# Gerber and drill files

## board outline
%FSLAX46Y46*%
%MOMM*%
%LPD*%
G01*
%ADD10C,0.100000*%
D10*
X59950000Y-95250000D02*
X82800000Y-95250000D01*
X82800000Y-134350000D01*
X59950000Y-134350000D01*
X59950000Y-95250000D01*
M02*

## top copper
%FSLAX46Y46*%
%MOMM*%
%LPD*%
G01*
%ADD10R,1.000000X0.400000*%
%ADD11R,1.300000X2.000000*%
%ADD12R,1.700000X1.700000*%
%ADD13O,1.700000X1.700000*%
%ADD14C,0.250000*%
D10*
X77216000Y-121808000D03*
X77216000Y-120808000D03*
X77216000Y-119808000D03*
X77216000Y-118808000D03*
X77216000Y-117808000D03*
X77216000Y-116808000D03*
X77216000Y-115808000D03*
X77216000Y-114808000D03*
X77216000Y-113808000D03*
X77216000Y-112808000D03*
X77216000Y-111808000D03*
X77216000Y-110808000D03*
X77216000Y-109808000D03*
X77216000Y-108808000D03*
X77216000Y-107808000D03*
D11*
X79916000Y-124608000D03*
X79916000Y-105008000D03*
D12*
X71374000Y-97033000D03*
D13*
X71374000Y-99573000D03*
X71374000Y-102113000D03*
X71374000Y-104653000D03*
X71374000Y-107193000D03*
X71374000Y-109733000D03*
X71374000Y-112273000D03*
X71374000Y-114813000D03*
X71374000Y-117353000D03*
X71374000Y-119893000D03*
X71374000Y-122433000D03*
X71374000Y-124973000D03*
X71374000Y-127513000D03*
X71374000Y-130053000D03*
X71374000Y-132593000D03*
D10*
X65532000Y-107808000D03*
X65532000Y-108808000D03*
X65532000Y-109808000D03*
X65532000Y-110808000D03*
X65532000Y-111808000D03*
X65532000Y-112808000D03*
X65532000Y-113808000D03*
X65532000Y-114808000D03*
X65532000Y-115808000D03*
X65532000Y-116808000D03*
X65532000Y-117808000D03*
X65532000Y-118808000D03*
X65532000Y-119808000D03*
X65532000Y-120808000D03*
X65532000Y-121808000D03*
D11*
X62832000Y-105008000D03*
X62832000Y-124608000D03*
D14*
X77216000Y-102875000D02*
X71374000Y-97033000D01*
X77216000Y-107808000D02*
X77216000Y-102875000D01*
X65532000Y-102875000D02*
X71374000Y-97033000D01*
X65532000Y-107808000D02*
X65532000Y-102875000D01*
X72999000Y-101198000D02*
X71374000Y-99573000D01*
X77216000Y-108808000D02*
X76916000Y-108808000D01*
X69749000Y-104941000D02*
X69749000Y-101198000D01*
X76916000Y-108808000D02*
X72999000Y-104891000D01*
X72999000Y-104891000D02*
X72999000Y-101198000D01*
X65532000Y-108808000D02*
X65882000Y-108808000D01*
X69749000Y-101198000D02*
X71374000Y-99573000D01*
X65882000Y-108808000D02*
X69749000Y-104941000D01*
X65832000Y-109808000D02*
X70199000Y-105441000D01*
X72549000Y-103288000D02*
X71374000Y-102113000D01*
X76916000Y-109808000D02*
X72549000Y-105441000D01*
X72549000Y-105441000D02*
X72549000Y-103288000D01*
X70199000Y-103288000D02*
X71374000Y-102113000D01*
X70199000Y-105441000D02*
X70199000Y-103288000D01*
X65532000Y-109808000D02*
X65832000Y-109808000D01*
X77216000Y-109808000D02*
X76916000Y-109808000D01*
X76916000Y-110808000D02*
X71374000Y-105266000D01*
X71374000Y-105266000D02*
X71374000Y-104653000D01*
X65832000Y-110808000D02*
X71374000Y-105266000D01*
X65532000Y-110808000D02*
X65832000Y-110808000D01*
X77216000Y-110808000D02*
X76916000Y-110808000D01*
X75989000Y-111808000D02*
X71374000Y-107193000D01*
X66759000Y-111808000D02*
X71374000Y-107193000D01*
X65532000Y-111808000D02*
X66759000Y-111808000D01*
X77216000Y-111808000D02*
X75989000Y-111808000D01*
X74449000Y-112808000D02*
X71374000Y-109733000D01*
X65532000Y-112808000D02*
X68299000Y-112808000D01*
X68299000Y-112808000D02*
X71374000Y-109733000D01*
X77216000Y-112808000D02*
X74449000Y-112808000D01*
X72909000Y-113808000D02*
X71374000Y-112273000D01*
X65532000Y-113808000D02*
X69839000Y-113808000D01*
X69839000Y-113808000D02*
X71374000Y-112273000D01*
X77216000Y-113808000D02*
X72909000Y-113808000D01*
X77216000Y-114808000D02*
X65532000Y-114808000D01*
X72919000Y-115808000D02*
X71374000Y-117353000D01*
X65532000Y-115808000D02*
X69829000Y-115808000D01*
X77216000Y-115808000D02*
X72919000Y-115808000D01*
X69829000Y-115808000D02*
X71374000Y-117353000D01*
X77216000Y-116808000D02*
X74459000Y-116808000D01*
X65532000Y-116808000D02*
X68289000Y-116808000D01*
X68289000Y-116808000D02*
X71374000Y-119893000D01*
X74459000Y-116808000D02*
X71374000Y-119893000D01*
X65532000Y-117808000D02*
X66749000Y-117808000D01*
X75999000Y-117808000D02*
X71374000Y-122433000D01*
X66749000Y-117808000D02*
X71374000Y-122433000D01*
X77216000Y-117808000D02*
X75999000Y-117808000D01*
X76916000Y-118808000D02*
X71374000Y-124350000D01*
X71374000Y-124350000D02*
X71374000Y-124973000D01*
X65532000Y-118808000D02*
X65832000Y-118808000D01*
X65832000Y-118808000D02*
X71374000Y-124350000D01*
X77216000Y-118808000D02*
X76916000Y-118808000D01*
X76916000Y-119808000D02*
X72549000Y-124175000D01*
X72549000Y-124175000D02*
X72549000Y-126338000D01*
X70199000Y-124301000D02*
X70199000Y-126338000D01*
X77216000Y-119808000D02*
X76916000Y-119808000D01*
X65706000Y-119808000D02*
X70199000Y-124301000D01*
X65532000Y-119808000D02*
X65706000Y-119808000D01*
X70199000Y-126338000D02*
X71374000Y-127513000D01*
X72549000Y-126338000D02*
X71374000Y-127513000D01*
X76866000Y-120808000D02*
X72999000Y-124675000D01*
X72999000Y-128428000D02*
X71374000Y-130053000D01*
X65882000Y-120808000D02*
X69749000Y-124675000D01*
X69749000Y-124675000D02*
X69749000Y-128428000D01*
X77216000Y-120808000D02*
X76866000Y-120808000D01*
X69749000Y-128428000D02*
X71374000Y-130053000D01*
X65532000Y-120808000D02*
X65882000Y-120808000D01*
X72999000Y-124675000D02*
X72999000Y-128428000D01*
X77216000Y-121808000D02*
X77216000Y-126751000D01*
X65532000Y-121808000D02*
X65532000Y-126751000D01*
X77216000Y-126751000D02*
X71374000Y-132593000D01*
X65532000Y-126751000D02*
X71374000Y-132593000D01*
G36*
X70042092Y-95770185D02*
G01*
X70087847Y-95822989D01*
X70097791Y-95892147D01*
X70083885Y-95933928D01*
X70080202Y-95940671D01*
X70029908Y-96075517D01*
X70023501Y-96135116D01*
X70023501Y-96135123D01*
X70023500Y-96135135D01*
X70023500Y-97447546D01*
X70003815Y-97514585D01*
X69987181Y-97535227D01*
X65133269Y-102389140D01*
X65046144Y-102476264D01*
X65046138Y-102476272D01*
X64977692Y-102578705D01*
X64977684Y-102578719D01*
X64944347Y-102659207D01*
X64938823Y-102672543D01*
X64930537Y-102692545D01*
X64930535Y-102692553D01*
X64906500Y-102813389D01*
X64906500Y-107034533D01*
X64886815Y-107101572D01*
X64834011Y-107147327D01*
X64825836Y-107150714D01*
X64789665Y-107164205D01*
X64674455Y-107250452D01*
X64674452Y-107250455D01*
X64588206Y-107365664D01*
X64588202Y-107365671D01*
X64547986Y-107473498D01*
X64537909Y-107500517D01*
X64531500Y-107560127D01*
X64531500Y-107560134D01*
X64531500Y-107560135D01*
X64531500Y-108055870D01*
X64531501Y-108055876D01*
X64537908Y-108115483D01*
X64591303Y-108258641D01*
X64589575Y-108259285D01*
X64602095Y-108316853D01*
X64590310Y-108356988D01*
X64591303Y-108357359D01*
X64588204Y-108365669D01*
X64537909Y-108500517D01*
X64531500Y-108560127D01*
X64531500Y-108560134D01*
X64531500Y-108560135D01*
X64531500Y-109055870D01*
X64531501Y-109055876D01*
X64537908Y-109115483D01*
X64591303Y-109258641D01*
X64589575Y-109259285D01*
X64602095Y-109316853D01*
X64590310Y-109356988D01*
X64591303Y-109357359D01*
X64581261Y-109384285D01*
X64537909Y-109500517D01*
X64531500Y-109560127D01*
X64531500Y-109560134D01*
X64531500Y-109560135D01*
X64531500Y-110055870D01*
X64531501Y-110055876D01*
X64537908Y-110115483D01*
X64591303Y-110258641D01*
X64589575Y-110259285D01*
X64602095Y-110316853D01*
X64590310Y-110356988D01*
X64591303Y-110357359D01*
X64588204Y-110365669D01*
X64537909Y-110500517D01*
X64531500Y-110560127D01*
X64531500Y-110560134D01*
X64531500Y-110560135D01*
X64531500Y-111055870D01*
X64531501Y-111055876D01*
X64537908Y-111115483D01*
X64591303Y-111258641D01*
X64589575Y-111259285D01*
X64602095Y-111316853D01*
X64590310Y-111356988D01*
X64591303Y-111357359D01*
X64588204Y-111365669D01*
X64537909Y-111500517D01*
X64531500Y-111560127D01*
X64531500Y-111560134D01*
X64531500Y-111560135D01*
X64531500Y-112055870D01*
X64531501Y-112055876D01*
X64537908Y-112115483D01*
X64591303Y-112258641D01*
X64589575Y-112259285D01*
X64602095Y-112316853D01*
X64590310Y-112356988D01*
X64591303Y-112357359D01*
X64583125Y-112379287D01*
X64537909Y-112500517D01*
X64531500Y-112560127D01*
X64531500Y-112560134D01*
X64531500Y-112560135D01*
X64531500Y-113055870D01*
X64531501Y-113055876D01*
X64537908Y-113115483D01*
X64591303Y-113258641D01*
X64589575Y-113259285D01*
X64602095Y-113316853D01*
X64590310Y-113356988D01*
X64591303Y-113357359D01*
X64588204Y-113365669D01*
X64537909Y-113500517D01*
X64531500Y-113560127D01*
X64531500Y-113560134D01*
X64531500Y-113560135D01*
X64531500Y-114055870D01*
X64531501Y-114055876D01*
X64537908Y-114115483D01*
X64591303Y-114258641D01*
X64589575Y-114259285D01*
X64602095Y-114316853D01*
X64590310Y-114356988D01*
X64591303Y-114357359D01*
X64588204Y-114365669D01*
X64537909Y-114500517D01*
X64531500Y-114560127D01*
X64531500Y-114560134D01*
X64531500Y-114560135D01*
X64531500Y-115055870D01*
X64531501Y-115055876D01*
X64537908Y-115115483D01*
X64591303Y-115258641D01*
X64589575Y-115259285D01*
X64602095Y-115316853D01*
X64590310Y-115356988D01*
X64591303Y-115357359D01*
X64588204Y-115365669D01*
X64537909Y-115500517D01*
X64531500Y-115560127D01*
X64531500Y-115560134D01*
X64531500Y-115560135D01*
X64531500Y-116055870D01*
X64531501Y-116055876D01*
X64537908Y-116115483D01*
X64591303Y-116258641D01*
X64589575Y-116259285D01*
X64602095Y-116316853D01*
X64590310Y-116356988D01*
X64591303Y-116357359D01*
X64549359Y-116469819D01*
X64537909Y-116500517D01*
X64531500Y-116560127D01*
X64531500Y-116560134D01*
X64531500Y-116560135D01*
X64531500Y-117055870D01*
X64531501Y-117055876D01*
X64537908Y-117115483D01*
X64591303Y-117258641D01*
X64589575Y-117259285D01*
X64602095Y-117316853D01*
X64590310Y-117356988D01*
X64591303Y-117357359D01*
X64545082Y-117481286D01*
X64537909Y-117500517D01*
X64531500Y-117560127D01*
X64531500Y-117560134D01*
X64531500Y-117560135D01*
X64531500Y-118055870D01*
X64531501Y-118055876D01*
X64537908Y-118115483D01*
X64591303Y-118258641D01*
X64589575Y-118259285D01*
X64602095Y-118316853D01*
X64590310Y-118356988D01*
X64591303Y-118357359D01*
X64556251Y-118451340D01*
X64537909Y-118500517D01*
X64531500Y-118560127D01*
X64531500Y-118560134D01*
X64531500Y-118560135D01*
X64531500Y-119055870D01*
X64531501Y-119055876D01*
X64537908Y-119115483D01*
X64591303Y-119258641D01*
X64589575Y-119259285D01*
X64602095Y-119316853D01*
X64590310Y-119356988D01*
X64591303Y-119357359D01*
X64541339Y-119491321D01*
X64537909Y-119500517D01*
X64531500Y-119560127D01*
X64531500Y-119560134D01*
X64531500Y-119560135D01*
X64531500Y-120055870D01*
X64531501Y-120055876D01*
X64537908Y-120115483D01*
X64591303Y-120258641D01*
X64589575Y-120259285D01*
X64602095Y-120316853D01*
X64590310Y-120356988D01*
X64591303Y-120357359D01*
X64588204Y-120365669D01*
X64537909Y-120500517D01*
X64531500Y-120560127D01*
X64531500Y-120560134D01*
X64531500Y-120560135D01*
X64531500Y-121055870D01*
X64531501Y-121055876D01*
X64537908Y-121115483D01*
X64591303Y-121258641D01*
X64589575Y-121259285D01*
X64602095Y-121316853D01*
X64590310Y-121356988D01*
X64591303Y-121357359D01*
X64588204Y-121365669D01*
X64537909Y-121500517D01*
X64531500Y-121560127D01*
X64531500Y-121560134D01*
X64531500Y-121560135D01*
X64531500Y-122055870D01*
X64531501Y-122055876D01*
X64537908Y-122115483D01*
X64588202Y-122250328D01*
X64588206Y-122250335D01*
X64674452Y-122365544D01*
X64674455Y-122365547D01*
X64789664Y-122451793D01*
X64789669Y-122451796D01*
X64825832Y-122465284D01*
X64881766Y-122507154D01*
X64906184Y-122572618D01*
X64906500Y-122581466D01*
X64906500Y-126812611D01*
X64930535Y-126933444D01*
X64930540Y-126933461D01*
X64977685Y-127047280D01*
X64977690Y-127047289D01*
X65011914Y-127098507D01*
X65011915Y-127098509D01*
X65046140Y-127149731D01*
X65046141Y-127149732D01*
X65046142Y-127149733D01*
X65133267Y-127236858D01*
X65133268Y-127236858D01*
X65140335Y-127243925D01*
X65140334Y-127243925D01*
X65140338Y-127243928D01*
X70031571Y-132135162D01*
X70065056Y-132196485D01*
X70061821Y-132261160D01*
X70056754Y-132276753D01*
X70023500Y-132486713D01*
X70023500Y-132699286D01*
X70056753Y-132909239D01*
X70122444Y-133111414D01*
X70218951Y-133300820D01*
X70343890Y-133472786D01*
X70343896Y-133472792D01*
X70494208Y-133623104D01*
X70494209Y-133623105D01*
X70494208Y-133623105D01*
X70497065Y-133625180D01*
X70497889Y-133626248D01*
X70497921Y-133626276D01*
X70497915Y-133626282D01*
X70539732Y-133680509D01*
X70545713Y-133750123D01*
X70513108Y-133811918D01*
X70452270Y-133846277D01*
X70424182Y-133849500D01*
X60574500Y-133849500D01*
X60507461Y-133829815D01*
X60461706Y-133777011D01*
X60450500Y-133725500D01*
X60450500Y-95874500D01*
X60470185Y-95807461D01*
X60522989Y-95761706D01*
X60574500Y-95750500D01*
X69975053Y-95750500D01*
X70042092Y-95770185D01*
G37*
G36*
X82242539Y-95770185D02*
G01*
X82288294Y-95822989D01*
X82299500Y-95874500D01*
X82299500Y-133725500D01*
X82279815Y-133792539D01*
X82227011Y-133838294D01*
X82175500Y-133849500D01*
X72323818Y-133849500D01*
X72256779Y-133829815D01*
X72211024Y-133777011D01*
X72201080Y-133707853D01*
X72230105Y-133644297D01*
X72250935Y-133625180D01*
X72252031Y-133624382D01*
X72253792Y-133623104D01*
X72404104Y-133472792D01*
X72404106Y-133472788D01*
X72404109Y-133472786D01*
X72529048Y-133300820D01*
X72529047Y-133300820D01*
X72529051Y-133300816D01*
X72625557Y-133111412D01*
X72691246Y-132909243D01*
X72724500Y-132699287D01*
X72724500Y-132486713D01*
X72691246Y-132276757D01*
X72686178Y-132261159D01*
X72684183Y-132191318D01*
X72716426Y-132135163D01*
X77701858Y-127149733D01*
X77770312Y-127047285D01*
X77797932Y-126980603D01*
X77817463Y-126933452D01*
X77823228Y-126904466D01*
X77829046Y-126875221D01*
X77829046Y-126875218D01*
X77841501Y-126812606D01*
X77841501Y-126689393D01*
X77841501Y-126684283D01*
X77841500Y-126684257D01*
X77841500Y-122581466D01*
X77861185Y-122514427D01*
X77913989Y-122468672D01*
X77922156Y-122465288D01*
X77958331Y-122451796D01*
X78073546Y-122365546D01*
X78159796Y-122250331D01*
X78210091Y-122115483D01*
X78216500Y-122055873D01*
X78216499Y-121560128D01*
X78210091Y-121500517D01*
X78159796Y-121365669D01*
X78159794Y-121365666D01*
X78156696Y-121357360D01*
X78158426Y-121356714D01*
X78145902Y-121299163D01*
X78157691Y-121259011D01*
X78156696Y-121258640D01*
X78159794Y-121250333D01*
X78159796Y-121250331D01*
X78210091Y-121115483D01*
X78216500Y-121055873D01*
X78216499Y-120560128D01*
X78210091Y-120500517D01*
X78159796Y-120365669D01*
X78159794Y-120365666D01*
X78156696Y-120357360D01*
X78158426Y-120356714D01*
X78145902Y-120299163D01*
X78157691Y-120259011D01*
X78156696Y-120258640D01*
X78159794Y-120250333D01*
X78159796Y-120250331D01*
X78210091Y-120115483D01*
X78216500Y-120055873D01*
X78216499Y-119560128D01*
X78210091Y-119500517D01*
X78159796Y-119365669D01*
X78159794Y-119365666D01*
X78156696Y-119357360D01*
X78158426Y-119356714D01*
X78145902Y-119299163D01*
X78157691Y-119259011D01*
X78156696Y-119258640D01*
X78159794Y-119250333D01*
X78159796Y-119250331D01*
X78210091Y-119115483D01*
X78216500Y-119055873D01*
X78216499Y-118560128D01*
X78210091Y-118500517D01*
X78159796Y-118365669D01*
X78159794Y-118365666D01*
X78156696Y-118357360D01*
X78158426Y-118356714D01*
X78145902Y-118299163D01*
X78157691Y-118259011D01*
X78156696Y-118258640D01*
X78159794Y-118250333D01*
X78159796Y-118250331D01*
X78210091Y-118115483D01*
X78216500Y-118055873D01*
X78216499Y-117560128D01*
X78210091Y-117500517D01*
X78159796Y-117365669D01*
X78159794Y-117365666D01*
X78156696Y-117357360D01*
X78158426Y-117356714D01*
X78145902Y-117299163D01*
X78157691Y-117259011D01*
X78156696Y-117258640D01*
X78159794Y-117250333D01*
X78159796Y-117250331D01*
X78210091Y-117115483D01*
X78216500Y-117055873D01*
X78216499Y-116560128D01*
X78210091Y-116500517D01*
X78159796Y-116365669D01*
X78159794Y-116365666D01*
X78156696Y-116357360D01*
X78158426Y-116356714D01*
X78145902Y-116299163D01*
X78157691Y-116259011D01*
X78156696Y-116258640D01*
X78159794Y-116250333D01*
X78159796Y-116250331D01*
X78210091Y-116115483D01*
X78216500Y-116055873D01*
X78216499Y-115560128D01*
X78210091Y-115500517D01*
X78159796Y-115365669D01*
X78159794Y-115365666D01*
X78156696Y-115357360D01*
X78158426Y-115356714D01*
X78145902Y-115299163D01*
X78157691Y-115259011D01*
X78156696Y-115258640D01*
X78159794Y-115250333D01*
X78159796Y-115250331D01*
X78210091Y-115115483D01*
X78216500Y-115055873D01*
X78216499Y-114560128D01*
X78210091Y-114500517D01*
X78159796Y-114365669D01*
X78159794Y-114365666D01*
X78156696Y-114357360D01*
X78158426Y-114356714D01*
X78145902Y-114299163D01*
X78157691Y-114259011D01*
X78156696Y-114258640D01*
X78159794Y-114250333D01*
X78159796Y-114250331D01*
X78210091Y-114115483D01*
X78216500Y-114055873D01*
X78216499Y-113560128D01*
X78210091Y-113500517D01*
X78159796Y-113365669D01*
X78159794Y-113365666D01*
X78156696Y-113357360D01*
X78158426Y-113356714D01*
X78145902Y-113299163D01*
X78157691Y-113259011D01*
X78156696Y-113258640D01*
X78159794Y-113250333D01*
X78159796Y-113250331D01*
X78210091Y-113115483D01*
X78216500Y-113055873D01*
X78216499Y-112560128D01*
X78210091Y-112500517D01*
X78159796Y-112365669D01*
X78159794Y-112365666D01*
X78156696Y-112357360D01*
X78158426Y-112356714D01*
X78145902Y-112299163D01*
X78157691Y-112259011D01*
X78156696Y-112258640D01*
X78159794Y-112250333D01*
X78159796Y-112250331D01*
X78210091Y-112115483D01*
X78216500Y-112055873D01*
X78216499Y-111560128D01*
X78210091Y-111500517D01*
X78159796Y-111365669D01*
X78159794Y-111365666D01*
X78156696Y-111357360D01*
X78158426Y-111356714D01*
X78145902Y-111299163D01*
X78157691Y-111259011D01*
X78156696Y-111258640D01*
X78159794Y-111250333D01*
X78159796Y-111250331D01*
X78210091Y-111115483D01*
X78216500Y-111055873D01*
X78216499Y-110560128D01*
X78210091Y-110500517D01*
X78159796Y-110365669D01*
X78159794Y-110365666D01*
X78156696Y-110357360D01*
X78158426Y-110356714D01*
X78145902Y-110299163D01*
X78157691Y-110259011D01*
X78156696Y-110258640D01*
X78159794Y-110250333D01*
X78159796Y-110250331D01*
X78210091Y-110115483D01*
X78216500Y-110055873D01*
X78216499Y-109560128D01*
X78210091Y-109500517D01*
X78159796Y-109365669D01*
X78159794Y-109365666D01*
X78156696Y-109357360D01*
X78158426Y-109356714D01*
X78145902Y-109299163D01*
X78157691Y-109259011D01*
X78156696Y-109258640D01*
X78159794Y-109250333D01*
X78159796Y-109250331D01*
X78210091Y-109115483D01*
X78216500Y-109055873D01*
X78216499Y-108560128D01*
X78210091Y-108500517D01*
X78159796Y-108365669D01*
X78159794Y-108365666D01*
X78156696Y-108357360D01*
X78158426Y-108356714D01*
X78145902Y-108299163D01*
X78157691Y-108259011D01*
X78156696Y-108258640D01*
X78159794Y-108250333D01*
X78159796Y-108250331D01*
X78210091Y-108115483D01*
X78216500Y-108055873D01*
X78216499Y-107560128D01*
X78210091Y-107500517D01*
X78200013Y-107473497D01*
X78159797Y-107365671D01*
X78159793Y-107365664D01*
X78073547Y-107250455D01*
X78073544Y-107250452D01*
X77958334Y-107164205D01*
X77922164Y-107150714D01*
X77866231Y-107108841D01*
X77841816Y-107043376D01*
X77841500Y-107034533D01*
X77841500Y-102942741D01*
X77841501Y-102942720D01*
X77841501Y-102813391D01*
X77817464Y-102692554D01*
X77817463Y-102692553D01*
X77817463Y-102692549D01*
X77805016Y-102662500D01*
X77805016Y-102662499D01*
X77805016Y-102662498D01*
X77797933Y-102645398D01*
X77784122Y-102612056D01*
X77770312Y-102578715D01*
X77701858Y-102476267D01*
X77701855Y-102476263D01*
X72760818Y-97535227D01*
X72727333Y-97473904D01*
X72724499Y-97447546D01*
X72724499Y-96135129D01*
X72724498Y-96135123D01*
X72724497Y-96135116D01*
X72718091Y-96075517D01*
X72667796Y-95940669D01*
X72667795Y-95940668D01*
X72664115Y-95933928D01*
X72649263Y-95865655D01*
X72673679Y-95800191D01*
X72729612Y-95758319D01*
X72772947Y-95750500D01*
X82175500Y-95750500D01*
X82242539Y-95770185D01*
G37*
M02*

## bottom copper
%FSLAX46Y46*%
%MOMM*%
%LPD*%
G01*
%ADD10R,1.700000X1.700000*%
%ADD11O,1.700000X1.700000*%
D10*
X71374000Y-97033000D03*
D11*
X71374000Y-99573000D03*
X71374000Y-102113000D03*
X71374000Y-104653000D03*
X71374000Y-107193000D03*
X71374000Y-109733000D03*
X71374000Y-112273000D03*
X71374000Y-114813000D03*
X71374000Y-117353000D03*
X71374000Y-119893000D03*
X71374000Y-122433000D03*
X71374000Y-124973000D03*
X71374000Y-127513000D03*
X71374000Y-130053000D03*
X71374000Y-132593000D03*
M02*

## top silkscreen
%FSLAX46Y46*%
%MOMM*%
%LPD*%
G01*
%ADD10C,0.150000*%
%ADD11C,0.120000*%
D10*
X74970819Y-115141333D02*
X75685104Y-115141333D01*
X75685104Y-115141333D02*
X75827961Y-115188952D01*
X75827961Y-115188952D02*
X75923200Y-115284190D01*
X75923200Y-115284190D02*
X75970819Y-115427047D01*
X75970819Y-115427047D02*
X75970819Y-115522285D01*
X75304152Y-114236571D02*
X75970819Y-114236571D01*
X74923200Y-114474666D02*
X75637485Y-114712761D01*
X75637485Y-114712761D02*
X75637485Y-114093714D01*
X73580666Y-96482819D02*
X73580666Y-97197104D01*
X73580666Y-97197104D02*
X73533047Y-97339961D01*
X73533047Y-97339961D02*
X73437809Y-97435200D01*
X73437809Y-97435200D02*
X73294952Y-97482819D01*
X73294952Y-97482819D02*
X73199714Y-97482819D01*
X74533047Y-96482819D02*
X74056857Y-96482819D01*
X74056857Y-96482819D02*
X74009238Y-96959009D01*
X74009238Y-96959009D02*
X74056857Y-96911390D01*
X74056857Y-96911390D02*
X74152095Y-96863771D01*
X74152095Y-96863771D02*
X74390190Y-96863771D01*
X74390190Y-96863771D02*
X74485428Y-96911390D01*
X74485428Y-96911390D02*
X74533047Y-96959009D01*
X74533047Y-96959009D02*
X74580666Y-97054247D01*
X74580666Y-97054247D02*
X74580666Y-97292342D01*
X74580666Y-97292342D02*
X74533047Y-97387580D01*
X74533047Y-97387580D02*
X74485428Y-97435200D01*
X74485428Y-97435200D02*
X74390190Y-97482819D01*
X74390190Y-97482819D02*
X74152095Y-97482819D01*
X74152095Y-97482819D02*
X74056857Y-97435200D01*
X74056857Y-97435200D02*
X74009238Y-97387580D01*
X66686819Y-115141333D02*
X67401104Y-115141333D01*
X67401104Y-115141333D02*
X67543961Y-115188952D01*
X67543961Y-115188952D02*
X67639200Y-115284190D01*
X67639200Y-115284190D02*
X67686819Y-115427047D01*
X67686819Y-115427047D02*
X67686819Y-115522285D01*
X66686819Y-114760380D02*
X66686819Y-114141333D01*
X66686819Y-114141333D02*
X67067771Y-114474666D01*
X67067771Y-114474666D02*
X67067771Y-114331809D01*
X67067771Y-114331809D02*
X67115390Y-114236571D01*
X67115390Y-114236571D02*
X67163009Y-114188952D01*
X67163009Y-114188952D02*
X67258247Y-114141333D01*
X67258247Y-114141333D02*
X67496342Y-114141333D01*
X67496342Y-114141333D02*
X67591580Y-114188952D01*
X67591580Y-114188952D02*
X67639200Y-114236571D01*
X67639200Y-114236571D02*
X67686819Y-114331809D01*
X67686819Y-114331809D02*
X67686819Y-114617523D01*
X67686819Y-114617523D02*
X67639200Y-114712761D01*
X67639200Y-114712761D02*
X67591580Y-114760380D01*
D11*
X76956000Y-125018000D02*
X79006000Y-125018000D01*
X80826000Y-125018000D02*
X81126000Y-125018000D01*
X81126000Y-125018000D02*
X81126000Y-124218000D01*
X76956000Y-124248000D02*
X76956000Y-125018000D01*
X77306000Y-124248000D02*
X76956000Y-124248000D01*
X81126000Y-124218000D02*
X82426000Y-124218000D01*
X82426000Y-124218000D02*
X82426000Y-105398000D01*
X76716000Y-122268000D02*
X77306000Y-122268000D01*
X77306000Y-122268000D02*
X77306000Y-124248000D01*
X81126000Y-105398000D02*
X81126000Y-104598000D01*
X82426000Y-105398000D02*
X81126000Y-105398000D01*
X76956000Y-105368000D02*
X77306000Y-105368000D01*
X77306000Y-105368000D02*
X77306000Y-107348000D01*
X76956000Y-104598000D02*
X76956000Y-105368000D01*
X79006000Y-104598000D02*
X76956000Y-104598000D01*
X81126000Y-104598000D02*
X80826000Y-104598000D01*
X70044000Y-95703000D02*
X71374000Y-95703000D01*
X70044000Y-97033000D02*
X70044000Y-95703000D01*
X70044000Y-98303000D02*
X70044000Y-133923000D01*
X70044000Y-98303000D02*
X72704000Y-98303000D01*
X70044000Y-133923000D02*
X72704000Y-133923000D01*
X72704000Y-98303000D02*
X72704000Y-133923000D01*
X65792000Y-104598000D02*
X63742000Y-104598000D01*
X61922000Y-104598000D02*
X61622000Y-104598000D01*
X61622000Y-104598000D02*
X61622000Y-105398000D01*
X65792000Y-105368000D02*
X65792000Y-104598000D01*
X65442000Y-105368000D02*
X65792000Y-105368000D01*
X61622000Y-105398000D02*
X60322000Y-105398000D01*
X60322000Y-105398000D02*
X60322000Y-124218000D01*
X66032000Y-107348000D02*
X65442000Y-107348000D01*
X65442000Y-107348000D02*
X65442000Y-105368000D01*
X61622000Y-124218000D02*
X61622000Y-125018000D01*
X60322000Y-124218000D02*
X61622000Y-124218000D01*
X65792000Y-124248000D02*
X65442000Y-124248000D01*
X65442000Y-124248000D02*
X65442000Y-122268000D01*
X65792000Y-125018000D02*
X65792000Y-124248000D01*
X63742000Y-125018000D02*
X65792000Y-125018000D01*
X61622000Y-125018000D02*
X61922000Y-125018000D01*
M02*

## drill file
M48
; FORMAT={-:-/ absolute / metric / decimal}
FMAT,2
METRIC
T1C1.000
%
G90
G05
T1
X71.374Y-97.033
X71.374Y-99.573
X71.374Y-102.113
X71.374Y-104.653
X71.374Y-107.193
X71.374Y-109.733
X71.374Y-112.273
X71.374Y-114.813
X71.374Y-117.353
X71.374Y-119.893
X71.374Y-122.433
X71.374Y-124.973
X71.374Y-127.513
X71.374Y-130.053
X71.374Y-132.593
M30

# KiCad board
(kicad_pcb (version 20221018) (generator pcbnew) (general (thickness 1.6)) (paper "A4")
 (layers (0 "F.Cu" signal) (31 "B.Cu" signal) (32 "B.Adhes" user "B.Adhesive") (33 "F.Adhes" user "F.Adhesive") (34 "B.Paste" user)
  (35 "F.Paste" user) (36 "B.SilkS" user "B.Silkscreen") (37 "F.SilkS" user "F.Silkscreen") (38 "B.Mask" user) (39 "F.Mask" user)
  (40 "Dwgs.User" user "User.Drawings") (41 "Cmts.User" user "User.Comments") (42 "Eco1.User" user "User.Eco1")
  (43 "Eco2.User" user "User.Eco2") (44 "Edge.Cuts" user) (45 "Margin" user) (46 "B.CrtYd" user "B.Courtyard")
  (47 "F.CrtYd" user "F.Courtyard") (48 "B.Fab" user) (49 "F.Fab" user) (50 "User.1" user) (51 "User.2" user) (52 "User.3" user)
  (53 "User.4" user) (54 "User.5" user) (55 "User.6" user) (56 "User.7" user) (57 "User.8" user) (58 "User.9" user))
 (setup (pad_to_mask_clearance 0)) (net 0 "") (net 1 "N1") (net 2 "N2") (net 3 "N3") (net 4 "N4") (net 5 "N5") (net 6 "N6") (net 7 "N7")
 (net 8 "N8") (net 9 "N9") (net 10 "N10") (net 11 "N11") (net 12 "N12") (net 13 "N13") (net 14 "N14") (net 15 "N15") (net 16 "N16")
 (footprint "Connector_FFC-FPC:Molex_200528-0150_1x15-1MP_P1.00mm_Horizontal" (layer "F.Cu") (at 78.126 114.808 90)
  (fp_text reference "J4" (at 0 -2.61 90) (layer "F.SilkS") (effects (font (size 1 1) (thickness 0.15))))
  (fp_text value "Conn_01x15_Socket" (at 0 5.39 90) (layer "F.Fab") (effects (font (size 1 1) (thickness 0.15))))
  (fp_line (start -10.21 -1.17) (end -10.21 0.88) (stroke (width 0.12) (type solid)) (layer "F.SilkS"))
  (fp_line (start -10.21 2.7) (end -10.21 3) (stroke (width 0.12) (type solid)) (layer "F.SilkS"))
  (fp_line (start -10.21 3) (end -9.41 3) (stroke (width 0.12) (type solid)) (layer "F.SilkS"))
  (fp_line (start -9.44 -1.17) (end -10.21 -1.17) (stroke (width 0.12) (type solid)) (layer "F.SilkS"))
  (fp_line (start -9.44 -0.82) (end -9.44 -1.17) (stroke (width 0.12) (type solid)) (layer "F.SilkS"))
  (fp_line (start -9.41 3) (end -9.41 4.3) (stroke (width 0.12) (type solid)) (layer "F.SilkS"))
  (fp_line (start -9.41 4.3) (end 9.41 4.3) (stroke (width 0.12) (type solid)) (layer "F.SilkS"))
  (fp_line (start -7.46 -1.41) (end -7.46 -0.82) (stroke (width 0.12) (type solid)) (layer "F.SilkS"))
  (fp_line (start -7.46 -0.82) (end -9.44 -0.82) (stroke (width 0.12) (type solid)) (layer "F.SilkS"))
  (fp_line (start 9.41 3) (end 10.21 3) (stroke (width 0.12) (type solid)) (layer "F.SilkS"))
  (fp_line (start 9.41 4.3) (end 9.41 3) (stroke (width 0.12) (type solid)) (layer "F.SilkS"))
  (fp_line (start 9.44 -1.17) (end 9.44 -0.82) (stroke (width 0.12) (type solid)) (layer "F.SilkS"))
  (fp_line (start 9.44 -0.82) (end 7.46 -0.82) (stroke (width 0.12) (type solid)) (layer "F.SilkS"))
  (fp_line (start 10.21 -1.17) (end 9.44 -1.17) (stroke (width 0.12) (type solid)) (layer "F.SilkS"))
  (fp_line (start 10.21 0.88) (end 10.21 -1.17) (stroke (width 0.12) (type solid)) (layer "F.SilkS"))
  (fp_line (start 10.21 3) (end 10.21 2.7) (stroke (width 0.12) (type solid)) (layer "F.SilkS"))
  (pad "1" smd rect (at -7 -0.91 90) (size 0.4 1) (layers "F.Cu" "F.Paste" "F.Mask") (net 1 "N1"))
  (pad "2" smd rect (at -6 -0.91 90) (size 0.4 1) (layers "F.Cu" "F.Paste" "F.Mask") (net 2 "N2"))
  (pad "3" smd rect (at -5 -0.91 90) (size 0.4 1) (layers "F.Cu" "F.Paste" "F.Mask") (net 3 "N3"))
  (pad "4" smd rect (at -4 -0.91 90) (size 0.4 1) (layers "F.Cu" "F.Paste" "F.Mask") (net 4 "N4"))
  (pad "5" smd rect (at -3 -0.91 90) (size 0.4 1) (layers "F.Cu" "F.Paste" "F.Mask") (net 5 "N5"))
  (pad "6" smd rect (at -2 -0.91 90) (size 0.4 1) (layers "F.Cu" "F.Paste" "F.Mask") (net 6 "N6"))
  (pad "7" smd rect (at -1 -0.91 90) (size 0.4 1) (layers "F.Cu" "F.Paste" "F.Mask") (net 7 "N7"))
  (pad "8" smd rect (at 0 -0.91 90) (size 0.4 1) (layers "F.Cu" "F.Paste" "F.Mask") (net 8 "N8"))
  (pad "9" smd rect (at 1 -0.91 90) (size 0.4 1) (layers "F.Cu" "F.Paste" "F.Mask") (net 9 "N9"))
  (pad "10" smd rect (at 2 -0.91 90) (size 0.4 1) (layers "F.Cu" "F.Paste" "F.Mask") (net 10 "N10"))
  (pad "11" smd rect (at 3 -0.91 90) (size 0.4 1) (layers "F.Cu" "F.Paste" "F.Mask") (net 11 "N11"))
  (pad "12" smd rect (at 4 -0.91 90) (size 0.4 1) (layers "F.Cu" "F.Paste" "F.Mask") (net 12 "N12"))
  (pad "13" smd rect (at 5 -0.91 90) (size 0.4 1) (layers "F.Cu" "F.Paste" "F.Mask") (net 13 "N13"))
  (pad "14" smd rect (at 6 -0.91 90) (size 0.4 1) (layers "F.Cu" "F.Paste" "F.Mask") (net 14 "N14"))
  (pad "15" smd rect (at 7 -0.91 90) (size 0.4 1) (layers "F.Cu" "F.Paste" "F.Mask") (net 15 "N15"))
  (pad "MP" smd rect (at -9.8 1.79 90) (size 2 1.3) (layers "F.Cu" "F.Paste" "F.Mask") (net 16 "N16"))
  (pad "MP" smd rect (at 9.8 1.79 90) (size 2 1.3) (layers "F.Cu" "F.Paste" "F.Mask") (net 16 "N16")))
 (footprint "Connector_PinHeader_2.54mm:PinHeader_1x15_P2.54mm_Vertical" (layer "F.Cu") (at 71.374 97.033)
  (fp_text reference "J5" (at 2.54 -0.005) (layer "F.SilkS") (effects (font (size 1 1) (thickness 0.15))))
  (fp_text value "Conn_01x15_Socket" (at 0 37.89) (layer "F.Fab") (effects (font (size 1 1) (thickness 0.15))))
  (fp_line (start -1.33 -1.33) (end 0 -1.33) (stroke (width 0.12) (type solid)) (layer "F.SilkS"))
  (fp_line (start -1.33 0) (end -1.33 -1.33) (stroke (width 0.12) (type solid)) (layer "F.SilkS"))
  (fp_line (start -1.33 1.27) (end -1.33 36.89) (stroke (width 0.12) (type solid)) (layer "F.SilkS"))
  (fp_line (start -1.33 1.27) (end 1.33 1.27) (stroke (width 0.12) (type solid)) (layer "F.SilkS"))
  (fp_line (start -1.33 36.89) (end 1.33 36.89) (stroke (width 0.12) (type solid)) (layer "F.SilkS"))
  (fp_line (start 1.33 1.27) (end 1.33 36.89) (stroke (width 0.12) (type solid)) (layer "F.SilkS"))
  (pad "1" thru_hole rect (at 0 0) (size 1.7 1.7) (drill 1) (layers "*.Cu" "*.Mask") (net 15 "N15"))
  (pad "2" thru_hole oval (at 0 2.54) (size 1.7 1.7) (drill 1) (layers "*.Cu" "*.Mask") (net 14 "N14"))
  (pad "3" thru_hole oval (at 0 5.08) (size 1.7 1.7) (drill 1) (layers "*.Cu" "*.Mask") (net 13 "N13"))
  (pad "4" thru_hole oval (at 0 7.62) (size 1.7 1.7) (drill 1) (layers "*.Cu" "*.Mask") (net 12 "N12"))
  (pad "5" thru_hole oval (at 0 10.16) (size 1.7 1.7) (drill 1) (layers "*.Cu" "*.Mask") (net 11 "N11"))
  (pad "6" thru_hole oval (at 0 12.7) (size 1.7 1.7) (drill 1) (layers "*.Cu" "*.Mask") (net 10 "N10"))
  (pad "7" thru_hole oval (at 0 15.24) (size 1.7 1.7) (drill 1) (layers "*.Cu" "*.Mask") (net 9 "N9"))
  (pad "8" thru_hole oval (at 0 17.78) (size 1.7 1.7) (drill 1) (layers "*.Cu" "*.Mask") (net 8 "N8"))
  (pad "9" thru_hole oval (at 0 20.32) (size 1.7 1.7) (drill 1) (layers "*.Cu" "*.Mask") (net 7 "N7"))
  (pad "10" thru_hole oval (at 0 22.86) (size 1.7 1.7) (drill 1) (layers "*.Cu" "*.Mask") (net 6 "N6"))
  (pad "11" thru_hole oval (at 0 25.4) (size 1.7 1.7) (drill 1) (layers "*.Cu" "*.Mask") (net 5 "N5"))
  (pad "12" thru_hole oval (at 0 27.94) (size 1.7 1.7) (drill 1) (layers "*.Cu" "*.Mask") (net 4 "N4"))
  (pad "13" thru_hole oval (at 0 30.48) (size 1.7 1.7) (drill 1) (layers "*.Cu" "*.Mask") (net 3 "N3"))
  (pad "14" thru_hole oval (at 0 33.02) (size 1.7 1.7) (drill 1) (layers "*.Cu" "*.Mask") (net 2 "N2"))
  (pad "15" thru_hole oval (at 0 35.56) (size 1.7 1.7) (drill 1) (layers "*.Cu" "*.Mask") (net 1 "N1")))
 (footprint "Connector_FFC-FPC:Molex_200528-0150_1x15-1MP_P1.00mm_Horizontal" (layer "F.Cu") (at 64.622 114.808 -90)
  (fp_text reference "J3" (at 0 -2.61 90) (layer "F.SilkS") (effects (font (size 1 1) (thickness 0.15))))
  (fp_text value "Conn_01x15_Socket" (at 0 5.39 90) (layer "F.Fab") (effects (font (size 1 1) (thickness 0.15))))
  (fp_line (start -10.21 -1.17) (end -10.21 0.88) (stroke (width 0.12) (type solid)) (layer "F.SilkS"))
  (fp_line (start -10.21 2.7) (end -10.21 3) (stroke (width 0.12) (type solid)) (layer "F.SilkS"))
  (fp_line (start -10.21 3) (end -9.41 3) (stroke (width 0.12) (type solid)) (layer "F.SilkS"))
  (fp_line (start -9.44 -1.17) (end -10.21 -1.17) (stroke (width 0.12) (type solid)) (layer "F.SilkS"))
  (fp_line (start -9.44 -0.82) (end -9.44 -1.17) (stroke (width 0.12) (type solid)) (layer "F.SilkS"))
  (fp_line (start -9.41 3) (end -9.41 4.3) (stroke (width 0.12) (type solid)) (layer "F.SilkS"))
  (fp_line (start -9.41 4.3) (end 9.41 4.3) (stroke (width 0.12) (type solid)) (layer "F.SilkS"))
  (fp_line (start -7.46 -1.41) (end -7.46 -0.82) (stroke (width 0.12) (type solid)) (layer "F.SilkS"))
  (fp_line (start -7.46 -0.82) (end -9.44 -0.82) (stroke (width 0.12) (type solid)) (layer "F.SilkS"))
  (fp_line (start 9.41 3) (end 10.21 3) (stroke (width 0.12) (type solid)) (layer "F.SilkS"))
  (fp_line (start 9.41 4.3) (end 9.41 3) (stroke (width 0.12) (type solid)) (layer "F.SilkS"))
  (fp_line (start 9.44 -1.17) (end 9.44 -0.82) (stroke (width 0.12) (type solid)) (layer "F.SilkS"))
  (fp_line (start 9.44 -0.82) (end 7.46 -0.82) (stroke (width 0.12) (type solid)) (layer "F.SilkS"))
  (fp_line (start 10.21 -1.17) (end 9.44 -1.17) (stroke (width 0.12) (type solid)) (layer "F.SilkS"))
  (fp_line (start 10.21 0.88) (end 10.21 -1.17) (stroke (width 0.12) (type solid)) (layer "F.SilkS"))
  (fp_line (start 10.21 3) (end 10.21 2.7) (stroke (width 0.12) (type solid)) (layer "F.SilkS"))
  (pad "1" smd rect (at -7 -0.91 270) (size 0.4 1) (layers "F.Cu" "F.Paste" "F.Mask") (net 15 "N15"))
  (pad "2" smd rect (at -6 -0.91 270) (size 0.4 1) (layers "F.Cu" "F.Paste" "F.Mask") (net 14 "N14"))
  (pad "3" smd rect (at -5 -0.91 270) (size 0.4 1) (layers "F.Cu" "F.Paste" "F.Mask") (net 13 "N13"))
  (pad "4" smd rect (at -4 -0.91 270) (size 0.4 1) (layers "F.Cu" "F.Paste" "F.Mask") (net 12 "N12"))
  (pad "5" smd rect (at -3 -0.91 270) (size 0.4 1) (layers "F.Cu" "F.Paste" "F.Mask") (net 11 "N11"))
  (pad "6" smd rect (at -2 -0.91 270) (size 0.4 1) (layers "F.Cu" "F.Paste" "F.Mask") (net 10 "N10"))
  (pad "7" smd rect (at -1 -0.91 270) (size 0.4 1) (layers "F.Cu" "F.Paste" "F.Mask") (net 9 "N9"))
  (pad "8" smd rect (at 0 -0.91 270) (size 0.4 1) (layers "F.Cu" "F.Paste" "F.Mask") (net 8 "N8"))
  (pad "9" smd rect (at 1 -0.91 270) (size 0.4 1) (layers "F.Cu" "F.Paste" "F.Mask") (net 7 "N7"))
  (pad "10" smd rect (at 2 -0.91 270) (size 0.4 1) (layers "F.Cu" "F.Paste" "F.Mask") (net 6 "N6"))
  (pad "11" smd rect (at 3 -0.91 270) (size 0.4 1) (layers "F.Cu" "F.Paste" "F.Mask") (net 5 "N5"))
  (pad "12" smd rect (at 4 -0.91 270) (size 0.4 1) (layers "F.Cu" "F.Paste" "F.Mask") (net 4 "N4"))
  (pad "13" smd rect (at 5 -0.91 270) (size 0.4 1) (layers "F.Cu" "F.Paste" "F.Mask") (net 3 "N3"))
  (pad "14" smd rect (at 6 -0.91 270) (size 0.4 1) (layers "F.Cu" "F.Paste" "F.Mask") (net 2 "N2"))
  (pad "15" smd rect (at 7 -0.91 270) (size 0.4 1) (layers "F.Cu" "F.Paste" "F.Mask") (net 1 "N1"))
  (pad "MP" smd rect (at -9.8 1.79 270) (size 2 1.3) (layers "F.Cu" "F.Paste" "F.Mask") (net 16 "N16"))
  (pad "MP" smd rect (at 9.8 1.79 270) (size 2 1.3) (layers "F.Cu" "F.Paste" "F.Mask") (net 16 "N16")))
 (gr_rect (start 59.95 95.25) (end 82.8 134.35) (stroke (width 0.1) (type default)) (fill none) (layer "Edge.Cuts"))
 (segment (start 77.216 102.875) (end 71.374 97.033) (width 0.25) (layer "F.Cu") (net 15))
 (segment (start 77.216 107.808) (end 77.216 102.875) (width 0.25) (layer "F.Cu") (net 15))
 (segment (start 65.532 102.875) (end 71.374 97.033) (width 0.25) (layer "F.Cu") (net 15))
 (segment (start 65.532 107.808) (end 65.532 102.875) (width 0.25) (layer "F.Cu") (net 15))
 (segment (start 72.999 101.198) (end 71.374 99.573) (width 0.25) (layer "F.Cu") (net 14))
 (segment (start 77.216 108.808) (end 76.916 108.808) (width 0.25) (layer "F.Cu") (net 14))
 (segment (start 69.749 104.941) (end 69.749 101.198) (width 0.25) (layer "F.Cu") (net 14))
 (segment (start 76.916 108.808) (end 72.999 104.891) (width 0.25) (layer "F.Cu") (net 14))
 (segment (start 72.999 104.891) (end 72.999 101.198) (width 0.25) (layer "F.Cu") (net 14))
 (segment (start 65.532 108.808) (end 65.882 108.808) (width 0.25) (layer "F.Cu") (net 14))
 (segment (start 69.749 101.198) (end 71.374 99.573) (width 0.25) (layer "F.Cu") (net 14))
 (segment (start 65.882 108.808) (end 69.749 104.941) (width 0.25) (layer "F.Cu") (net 14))
 (segment (start 65.832 109.808) (end 70.199 105.441) (width 0.25) (layer "F.Cu") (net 13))
 (segment (start 72.549 103.288) (end 71.374 102.113) (width 0.25) (layer "F.Cu") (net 13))
 (segment (start 76.916 109.808) (end 72.549 105.441) (width 0.25) (layer "F.Cu") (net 13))
 (segment (start 72.549 105.441) (end 72.549 103.288) (width 0.25) (layer "F.Cu") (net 13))
 (segment (start 70.199 103.288) (end 71.374 102.113) (width 0.25) (layer "F.Cu") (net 13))
 (segment (start 70.199 105.441) (end 70.199 103.288) (width 0.25) (layer "F.Cu") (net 13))
 (segment (start 65.532 109.808) (end 65.832 109.808) (width 0.25) (layer "F.Cu") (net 13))
 (segment (start 77.216 109.808) (end 76.916 109.808) (width 0.25) (layer "F.Cu") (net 13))
 (segment (start 76.916 110.808) (end 71.374 105.266) (width 0.25) (layer "F.Cu") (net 12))
 (segment (start 71.374 105.266) (end 71.374 104.653) (width 0.25) (layer "F.Cu") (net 12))
 (segment (start 65.832 110.808) (end 71.374 105.266) (width 0.25) (layer "F.Cu") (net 12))
 (segment (start 65.532 110.808) (end 65.832 110.808) (width 0.25) (layer "F.Cu") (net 12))
 (segment (start 77.216 110.808) (end 76.916 110.808) (width 0.25) (layer "F.Cu") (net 12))
 (segment (start 75.989 111.808) (end 71.374 107.193) (width 0.25) (layer "F.Cu") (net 11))
 (segment (start 66.759 111.808) (end 71.374 107.193) (width 0.25) (layer "F.Cu") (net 11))
 (segment (start 65.532 111.808) (end 66.759 111.808) (width 0.25) (layer "F.Cu") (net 11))
 (segment (start 77.216 111.808) (end 75.989 111.808) (width 0.25) (layer "F.Cu") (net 11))
 (segment (start 74.449 112.808) (end 71.374 109.733) (width 0.25) (layer "F.Cu") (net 10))
 (segment (start 65.532 112.808) (end 68.299 112.808) (width 0.25) (layer "F.Cu") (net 10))
 (segment (start 68.299 112.808) (end 71.374 109.733) (width 0.25) (layer "F.Cu") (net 10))
 (segment (start 77.216 112.808) (end 74.449 112.808) (width 0.25) (layer "F.Cu") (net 10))
 (segment (start 72.909 113.808) (end 71.374 112.273) (width 0.25) (layer "F.Cu") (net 9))
 (segment (start 65.532 113.808) (end 69.839 113.808) (width 0.25) (layer "F.Cu") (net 9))
 (segment (start 69.839 113.808) (end 71.374 112.273) (width 0.25) (layer "F.Cu") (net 9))
 (segment (start 77.216 113.808) (end 72.909 113.808) (width 0.25) (layer "F.Cu") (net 9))
 (segment (start 77.216 114.808) (end 65.532 114.808) (width 0.25) (layer "F.Cu") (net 8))
 (segment (start 72.919 115.808) (end 71.374 117.353) (width 0.25) (layer "F.Cu") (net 7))
 (segment (start 65.532 115.808) (end 69.829 115.808) (width 0.25) (layer "F.Cu") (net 7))
 (segment (start 77.216 115.808) (end 72.919 115.808) (width 0.25) (layer "F.Cu") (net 7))
 (segment (start 69.829 115.808) (end 71.374 117.353) (width 0.25) (layer "F.Cu") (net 7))
 (segment (start 77.216 116.808) (end 74.459 116.808) (width 0.25) (layer "F.Cu") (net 6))
 (segment (start 65.532 116.808) (end 68.289 116.808) (width 0.25) (layer "F.Cu") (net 6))
 (segment (start 68.289 116.808) (end 71.374 119.893) (width 0.25) (layer "F.Cu") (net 6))
 (segment (start 74.459 116.808) (end 71.374 119.893) (width 0.25) (layer "F.Cu") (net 6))
 (segment (start 65.532 117.808) (end 66.749 117.808) (width 0.25) (layer "F.Cu") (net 5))
 (segment (start 75.999 117.808) (end 71.374 122.433) (width 0.25) (layer "F.Cu") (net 5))
 (segment (start 66.749 117.808) (end 71.374 122.433) (width 0.25) (layer "F.Cu") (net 5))
 (segment (start 77.216 117.808) (end 75.999 117.808) (width 0.25) (layer "F.Cu") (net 5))
 (segment (start 76.916 118.808) (end 71.374 124.35) (width 0.25) (layer "F.Cu") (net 4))
 (segment (start 71.374 124.35) (end 71.374 124.973) (width 0.25) (layer "F.Cu") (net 4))
 (segment (start 65.532 118.808) (end 65.832 118.808) (width 0.25) (layer "F.Cu") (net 4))
 (segment (start 65.832 118.808) (end 71.374 124.35) (width 0.25) (layer "F.Cu") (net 4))
 (segment (start 77.216 118.808) (end 76.916 118.808) (width 0.25) (layer "F.Cu") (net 4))
 (segment (start 76.916 119.808) (end 72.549 124.175) (width 0.25) (layer "F.Cu") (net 3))
 (segment (start 72.549 124.175) (end 72.549 126.338) (width 0.25) (layer "F.Cu") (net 3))
 (segment (start 70.199 124.301) (end 70.199 126.338) (width 0.25) (layer "F.Cu") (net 3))
 (segment (start 77.216 119.808) (end 76.916 119.808) (width 0.25) (layer "F.Cu") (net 3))
 (segment (start 65.706 119.808) (end 70.199 124.301) (width 0.25) (layer "F.Cu") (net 3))
 (segment (start 65.532 119.808) (end 65.706 119.808) (width 0.25) (layer "F.Cu") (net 3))
 (segment (start 70.199 126.338) (end 71.374 127.513) (width 0.25) (layer "F.Cu") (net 3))
 (segment (start 72.549 126.338) (end 71.374 127.513) (width 0.25) (layer "F.Cu") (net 3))
 (segment (start 76.866 120.808) (end 72.999 124.675) (width 0.25) (layer "F.Cu") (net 2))
 (segment (start 72.999 128.428) (end 71.374 130.053) (width 0.25) (layer "F.Cu") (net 2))
 (segment (start 65.882 120.808) (end 69.749 124.675) (width 0.25) (layer "F.Cu") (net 2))
 (segment (start 69.749 124.675) (end 69.749 128.428) (width 0.25) (layer "F.Cu") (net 2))
 (segment (start 77.216 120.808) (end 76.866 120.808) (width 0.25) (layer "F.Cu") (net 2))
 (segment (start 69.749 128.428) (end 71.374 130.053) (width 0.25) (layer "F.Cu") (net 2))
 (segment (start 65.532 120.808) (end 65.882 120.808) (width 0.25) (layer "F.Cu") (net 2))
 (segment (start 72.999 124.675) (end 72.999 128.428) (width 0.25) (layer "F.Cu") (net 2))
 (segment (start 77.216 121.808) (end 77.216 126.751) (width 0.25) (layer "F.Cu") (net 1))
 (segment (start 65.532 121.808) (end 65.532 126.751) (width 0.25) (layer "F.Cu") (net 1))
 (segment (start 77.216 126.751) (end 71.374 132.593) (width 0.25) (layer "F.Cu") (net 1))
 (segment (start 65.532 126.751) (end 71.374 132.593) (width 0.25) (layer "F.Cu") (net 1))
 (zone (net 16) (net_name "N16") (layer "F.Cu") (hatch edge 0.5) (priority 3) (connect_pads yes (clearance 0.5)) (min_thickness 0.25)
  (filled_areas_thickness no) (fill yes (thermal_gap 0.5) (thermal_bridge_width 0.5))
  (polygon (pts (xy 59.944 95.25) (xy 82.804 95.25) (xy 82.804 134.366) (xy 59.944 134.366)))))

